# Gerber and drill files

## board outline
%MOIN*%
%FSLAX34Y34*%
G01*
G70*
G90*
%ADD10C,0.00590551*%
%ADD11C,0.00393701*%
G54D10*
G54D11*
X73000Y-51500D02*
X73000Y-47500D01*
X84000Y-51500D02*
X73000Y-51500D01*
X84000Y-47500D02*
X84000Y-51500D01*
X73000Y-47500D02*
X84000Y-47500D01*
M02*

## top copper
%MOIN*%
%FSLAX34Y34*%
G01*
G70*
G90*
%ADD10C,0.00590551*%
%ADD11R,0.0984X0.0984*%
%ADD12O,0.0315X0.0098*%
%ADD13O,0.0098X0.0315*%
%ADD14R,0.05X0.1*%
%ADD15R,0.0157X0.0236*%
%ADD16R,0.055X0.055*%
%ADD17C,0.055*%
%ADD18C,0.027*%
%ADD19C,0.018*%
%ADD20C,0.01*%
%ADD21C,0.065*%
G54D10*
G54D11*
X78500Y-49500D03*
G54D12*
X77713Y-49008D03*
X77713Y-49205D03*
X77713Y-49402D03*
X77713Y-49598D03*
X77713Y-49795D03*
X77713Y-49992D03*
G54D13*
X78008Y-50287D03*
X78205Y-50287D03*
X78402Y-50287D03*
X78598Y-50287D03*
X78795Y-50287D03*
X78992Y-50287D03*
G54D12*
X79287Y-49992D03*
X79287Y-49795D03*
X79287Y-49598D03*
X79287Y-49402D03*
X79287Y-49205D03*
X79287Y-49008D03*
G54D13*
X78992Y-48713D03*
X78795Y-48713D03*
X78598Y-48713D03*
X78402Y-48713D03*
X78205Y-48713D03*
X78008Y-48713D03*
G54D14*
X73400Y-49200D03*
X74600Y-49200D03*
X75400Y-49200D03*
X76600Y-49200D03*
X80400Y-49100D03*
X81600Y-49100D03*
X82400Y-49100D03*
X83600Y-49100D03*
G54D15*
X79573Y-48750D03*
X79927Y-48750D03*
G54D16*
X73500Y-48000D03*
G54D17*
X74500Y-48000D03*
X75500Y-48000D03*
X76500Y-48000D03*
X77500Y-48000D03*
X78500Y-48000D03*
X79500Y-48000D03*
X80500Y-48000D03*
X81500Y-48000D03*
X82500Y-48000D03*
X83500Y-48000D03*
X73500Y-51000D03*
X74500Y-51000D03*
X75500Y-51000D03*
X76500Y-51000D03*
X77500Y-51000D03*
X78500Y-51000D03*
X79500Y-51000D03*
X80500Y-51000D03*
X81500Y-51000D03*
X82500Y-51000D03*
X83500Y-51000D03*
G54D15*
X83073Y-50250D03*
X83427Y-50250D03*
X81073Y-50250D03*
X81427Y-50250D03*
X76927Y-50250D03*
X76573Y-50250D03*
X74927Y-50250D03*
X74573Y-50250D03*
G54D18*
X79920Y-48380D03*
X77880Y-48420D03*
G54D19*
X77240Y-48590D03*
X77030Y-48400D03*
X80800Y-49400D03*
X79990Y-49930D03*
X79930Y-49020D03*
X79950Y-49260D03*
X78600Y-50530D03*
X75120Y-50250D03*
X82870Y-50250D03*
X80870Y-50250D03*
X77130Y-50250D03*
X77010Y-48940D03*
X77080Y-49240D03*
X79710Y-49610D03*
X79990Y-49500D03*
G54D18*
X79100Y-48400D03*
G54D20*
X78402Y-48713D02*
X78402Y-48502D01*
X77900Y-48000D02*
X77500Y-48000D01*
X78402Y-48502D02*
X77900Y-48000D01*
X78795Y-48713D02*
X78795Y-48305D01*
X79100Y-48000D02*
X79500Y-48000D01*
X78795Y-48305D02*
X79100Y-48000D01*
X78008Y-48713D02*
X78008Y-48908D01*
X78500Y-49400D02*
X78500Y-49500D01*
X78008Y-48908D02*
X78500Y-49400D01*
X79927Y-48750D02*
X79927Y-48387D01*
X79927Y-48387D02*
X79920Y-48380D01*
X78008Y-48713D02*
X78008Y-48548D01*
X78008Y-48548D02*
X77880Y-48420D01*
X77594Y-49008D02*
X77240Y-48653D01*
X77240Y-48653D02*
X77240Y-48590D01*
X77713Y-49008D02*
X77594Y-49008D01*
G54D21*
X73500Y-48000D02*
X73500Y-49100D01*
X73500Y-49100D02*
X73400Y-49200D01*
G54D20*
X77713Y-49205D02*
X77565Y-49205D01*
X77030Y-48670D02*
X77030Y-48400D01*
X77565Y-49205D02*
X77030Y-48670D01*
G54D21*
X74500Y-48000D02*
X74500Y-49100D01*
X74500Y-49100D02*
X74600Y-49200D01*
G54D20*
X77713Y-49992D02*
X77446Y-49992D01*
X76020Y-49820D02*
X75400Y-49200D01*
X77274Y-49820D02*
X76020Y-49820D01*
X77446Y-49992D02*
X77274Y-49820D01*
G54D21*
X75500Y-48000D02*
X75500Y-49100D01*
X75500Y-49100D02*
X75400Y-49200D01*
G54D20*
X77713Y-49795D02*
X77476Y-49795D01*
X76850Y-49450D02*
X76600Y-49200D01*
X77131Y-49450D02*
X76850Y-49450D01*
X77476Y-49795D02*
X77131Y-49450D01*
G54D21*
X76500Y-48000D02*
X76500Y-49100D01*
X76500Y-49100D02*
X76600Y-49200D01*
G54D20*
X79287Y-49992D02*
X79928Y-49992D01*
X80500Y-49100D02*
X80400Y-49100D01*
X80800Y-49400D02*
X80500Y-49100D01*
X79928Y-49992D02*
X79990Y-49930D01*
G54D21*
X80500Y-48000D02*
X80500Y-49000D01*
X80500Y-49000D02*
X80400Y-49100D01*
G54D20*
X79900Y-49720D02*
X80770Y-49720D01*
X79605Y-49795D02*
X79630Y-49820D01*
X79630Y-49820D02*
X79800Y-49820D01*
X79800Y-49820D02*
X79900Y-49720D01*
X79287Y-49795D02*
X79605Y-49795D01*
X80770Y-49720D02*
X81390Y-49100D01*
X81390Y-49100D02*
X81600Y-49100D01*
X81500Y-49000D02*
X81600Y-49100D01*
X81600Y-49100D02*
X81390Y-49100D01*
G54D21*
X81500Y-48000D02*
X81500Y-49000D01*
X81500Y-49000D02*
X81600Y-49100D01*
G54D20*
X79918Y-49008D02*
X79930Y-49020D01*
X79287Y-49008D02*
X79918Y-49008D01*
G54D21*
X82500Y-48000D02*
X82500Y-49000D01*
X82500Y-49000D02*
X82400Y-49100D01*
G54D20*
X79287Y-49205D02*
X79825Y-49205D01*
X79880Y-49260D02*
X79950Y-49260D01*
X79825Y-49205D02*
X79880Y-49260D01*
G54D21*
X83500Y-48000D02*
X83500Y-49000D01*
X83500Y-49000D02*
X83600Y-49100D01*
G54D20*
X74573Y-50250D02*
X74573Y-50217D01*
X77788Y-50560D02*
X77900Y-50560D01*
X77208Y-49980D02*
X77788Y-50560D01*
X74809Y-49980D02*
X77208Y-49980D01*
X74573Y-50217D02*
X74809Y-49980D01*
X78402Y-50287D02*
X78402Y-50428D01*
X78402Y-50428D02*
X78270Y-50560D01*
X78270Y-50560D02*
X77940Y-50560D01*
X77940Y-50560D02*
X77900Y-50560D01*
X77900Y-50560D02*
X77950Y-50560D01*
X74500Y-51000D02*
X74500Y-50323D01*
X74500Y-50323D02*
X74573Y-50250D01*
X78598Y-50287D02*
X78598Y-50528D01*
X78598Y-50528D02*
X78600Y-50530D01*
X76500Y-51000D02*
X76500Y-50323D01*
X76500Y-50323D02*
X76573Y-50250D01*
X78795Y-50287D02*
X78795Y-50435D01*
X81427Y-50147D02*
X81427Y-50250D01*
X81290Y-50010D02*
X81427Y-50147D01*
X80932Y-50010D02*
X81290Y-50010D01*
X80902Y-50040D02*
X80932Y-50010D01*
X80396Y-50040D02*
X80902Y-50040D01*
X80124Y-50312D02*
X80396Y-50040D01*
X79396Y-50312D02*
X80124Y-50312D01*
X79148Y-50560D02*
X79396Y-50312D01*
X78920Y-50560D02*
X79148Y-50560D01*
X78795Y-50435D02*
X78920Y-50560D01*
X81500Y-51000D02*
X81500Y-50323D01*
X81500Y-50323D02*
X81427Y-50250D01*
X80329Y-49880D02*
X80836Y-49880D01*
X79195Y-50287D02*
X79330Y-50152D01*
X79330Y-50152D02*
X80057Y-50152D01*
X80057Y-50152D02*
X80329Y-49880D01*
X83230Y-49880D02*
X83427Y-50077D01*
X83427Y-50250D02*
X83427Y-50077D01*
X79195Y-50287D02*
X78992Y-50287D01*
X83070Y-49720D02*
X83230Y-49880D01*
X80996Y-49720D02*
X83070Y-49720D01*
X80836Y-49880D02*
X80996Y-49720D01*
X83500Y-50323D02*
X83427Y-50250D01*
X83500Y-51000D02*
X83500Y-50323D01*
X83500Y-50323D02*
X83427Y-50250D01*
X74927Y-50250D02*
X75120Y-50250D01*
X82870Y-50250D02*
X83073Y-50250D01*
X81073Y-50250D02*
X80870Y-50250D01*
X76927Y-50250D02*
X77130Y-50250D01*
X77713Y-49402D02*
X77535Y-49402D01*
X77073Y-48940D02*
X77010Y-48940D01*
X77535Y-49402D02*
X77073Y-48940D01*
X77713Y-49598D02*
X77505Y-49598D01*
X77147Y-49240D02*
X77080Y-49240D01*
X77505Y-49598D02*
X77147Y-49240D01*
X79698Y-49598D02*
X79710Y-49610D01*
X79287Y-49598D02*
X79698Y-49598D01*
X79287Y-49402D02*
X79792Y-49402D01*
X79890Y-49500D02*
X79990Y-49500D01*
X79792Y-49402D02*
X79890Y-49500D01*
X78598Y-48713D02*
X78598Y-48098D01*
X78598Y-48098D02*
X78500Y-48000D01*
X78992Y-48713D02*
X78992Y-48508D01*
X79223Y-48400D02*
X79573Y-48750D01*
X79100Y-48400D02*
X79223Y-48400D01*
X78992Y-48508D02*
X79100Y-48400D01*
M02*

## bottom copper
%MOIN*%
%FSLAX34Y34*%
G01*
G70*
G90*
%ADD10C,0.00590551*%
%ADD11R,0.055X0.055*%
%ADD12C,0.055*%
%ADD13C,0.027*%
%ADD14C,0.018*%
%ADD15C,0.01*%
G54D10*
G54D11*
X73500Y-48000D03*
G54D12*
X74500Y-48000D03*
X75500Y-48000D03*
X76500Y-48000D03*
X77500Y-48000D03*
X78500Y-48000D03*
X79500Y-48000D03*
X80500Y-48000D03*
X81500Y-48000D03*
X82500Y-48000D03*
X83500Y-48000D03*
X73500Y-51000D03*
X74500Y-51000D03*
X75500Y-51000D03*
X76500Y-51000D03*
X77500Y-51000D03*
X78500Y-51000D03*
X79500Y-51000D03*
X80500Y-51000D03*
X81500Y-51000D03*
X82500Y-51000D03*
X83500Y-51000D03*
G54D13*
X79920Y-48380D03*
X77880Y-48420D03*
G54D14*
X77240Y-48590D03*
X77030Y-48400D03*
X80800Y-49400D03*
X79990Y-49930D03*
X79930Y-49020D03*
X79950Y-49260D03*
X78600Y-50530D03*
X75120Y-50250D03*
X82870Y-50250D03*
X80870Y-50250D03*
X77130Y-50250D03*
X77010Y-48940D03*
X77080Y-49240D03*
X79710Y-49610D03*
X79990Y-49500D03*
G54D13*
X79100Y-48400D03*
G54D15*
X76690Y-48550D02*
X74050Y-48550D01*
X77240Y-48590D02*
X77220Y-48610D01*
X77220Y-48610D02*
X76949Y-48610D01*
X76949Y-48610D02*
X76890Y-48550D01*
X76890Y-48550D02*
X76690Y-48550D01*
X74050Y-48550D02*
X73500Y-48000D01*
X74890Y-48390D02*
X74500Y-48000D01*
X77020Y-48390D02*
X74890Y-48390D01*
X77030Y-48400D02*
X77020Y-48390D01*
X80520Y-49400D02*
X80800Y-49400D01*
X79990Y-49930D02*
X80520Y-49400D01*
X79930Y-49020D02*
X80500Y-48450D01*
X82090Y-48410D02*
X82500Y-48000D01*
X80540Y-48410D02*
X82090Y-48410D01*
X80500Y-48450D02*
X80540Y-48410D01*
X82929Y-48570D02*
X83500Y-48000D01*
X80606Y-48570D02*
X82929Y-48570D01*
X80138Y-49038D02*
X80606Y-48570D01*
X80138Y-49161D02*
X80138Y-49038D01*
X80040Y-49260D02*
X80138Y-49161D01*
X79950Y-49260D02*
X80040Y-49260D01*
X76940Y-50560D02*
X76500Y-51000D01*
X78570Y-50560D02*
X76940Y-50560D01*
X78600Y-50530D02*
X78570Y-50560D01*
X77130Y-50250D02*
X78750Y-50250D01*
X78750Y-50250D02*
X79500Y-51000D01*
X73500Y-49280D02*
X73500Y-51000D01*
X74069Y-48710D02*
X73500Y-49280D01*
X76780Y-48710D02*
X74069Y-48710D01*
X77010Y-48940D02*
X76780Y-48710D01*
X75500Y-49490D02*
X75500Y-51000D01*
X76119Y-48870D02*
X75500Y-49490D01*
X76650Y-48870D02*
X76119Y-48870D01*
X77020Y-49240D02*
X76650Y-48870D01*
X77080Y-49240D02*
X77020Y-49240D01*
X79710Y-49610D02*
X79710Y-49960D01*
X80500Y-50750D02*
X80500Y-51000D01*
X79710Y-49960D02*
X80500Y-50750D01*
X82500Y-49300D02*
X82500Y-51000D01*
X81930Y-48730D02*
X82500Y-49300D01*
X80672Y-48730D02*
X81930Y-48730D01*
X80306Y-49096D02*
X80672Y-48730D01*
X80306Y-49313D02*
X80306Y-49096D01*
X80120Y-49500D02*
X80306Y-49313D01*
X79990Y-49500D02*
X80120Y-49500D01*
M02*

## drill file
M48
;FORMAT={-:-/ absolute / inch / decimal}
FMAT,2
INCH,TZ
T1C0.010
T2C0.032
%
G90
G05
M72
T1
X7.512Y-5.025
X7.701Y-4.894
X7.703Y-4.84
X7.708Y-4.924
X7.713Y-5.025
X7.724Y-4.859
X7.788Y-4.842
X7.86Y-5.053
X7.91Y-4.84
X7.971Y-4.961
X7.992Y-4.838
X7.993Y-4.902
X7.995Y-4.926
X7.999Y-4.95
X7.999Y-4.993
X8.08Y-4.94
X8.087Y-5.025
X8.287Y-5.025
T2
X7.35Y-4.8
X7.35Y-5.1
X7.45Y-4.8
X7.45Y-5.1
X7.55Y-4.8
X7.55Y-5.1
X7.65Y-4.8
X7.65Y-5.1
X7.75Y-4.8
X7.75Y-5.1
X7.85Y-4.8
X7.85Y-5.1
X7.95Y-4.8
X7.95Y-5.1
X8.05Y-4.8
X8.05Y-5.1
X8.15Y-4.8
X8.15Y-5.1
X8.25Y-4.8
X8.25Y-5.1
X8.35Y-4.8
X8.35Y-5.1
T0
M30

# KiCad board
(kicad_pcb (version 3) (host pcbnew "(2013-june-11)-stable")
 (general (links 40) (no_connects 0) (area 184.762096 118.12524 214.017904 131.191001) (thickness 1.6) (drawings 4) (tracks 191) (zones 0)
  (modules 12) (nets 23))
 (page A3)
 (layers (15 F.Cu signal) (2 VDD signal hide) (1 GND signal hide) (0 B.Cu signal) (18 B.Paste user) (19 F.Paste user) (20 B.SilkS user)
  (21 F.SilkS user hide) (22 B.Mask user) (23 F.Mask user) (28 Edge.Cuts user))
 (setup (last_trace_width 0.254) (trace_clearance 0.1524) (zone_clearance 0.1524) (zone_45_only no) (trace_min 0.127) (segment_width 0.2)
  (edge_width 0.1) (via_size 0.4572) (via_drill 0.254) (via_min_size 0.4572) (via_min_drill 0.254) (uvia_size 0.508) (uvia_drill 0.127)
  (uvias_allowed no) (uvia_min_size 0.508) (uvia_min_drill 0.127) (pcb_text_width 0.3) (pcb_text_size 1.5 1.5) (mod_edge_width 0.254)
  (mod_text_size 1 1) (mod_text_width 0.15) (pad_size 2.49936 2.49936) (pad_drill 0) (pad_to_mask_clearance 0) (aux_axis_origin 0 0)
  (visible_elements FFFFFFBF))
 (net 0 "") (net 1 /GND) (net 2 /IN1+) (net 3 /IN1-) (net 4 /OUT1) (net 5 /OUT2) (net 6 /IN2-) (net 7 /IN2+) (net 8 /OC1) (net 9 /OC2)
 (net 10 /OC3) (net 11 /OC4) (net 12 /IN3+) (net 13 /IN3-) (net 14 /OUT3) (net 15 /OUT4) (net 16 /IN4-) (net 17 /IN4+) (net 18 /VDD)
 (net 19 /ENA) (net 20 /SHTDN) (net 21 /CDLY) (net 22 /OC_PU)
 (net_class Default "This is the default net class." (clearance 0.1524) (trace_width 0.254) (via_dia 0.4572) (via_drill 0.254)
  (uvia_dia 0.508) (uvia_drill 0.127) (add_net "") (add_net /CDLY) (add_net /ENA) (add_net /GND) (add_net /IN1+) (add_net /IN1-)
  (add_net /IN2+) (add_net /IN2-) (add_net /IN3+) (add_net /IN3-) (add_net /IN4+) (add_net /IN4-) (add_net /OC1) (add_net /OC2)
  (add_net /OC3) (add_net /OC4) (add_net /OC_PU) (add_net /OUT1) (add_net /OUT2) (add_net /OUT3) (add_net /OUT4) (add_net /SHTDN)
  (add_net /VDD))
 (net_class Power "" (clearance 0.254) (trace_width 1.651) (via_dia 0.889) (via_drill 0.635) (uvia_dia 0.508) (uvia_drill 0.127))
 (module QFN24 (layer F.Cu) (at 199.39 125.73) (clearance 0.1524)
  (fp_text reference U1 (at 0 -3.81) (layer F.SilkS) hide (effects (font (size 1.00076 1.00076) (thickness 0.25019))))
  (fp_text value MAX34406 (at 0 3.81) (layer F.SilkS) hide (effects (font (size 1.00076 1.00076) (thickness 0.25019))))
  (pad 25 smd rect (at 0 0 270) (size 2.49936 2.49936) (layers F.Cu F.Paste F.Mask) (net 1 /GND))
  (pad 1 smd oval (at -1.99898 -1.24968) (size 0.8001 0.24892) (layers F.Cu F.Paste F.Mask) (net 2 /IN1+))
  (pad 2 smd oval (at -1.99898 -0.7493) (size 0.8001 0.24892) (layers F.Cu F.Paste F.Mask) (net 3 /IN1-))
  (pad 3 smd oval (at -1.99898 -0.24892) (size 0.8001 0.24892) (layers F.Cu F.Paste F.Mask) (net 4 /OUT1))
  (pad 4 smd oval (at -1.99898 0.24892) (size 0.8001 0.24892) (layers F.Cu F.Paste F.Mask) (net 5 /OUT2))
  (pad 5 smd oval (at -1.99898 0.7493) (size 0.8001 0.24892) (layers F.Cu F.Paste F.Mask) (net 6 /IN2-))
  (pad 6 smd oval (at -1.99898 1.24968) (size 0.8001 0.24892) (layers F.Cu F.Paste F.Mask) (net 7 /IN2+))
  (pad 7 smd oval (at -1.24968 1.99898 90) (size 0.8001 0.24892) (layers F.Cu F.Paste F.Mask))
  (pad 8 smd oval (at -0.7493 1.99898 90) (size 0.8001 0.24892) (layers F.Cu F.Paste F.Mask))
  (pad 9 smd oval (at -0.24892 1.99898 90) (size 0.8001 0.24892) (layers F.Cu F.Paste F.Mask) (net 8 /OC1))
  (pad 10 smd oval (at 0.24892 1.99898 90) (size 0.8001 0.24892) (layers F.Cu F.Paste F.Mask) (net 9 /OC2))
  (pad 11 smd oval (at 0.7493 1.99898 90) (size 0.8001 0.24892) (layers F.Cu F.Paste F.Mask) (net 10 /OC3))
  (pad 12 smd oval (at 1.24968 1.99898 90) (size 0.8001 0.24892) (layers F.Cu F.Paste F.Mask) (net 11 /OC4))
  (pad 13 smd oval (at 1.99898 1.24968 180) (size 0.8001 0.24892) (layers F.Cu F.Paste F.Mask) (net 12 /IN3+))
  (pad 14 smd oval (at 1.99898 0.7493 180) (size 0.8001 0.24892) (layers F.Cu F.Paste F.Mask) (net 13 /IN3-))
  (pad 15 smd oval (at 1.99898 0.24892 180) (size 0.8001 0.24892) (layers F.Cu F.Paste F.Mask) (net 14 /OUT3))
  (pad 16 smd oval (at 1.99898 -0.24892 180) (size 0.8001 0.24892) (layers F.Cu F.Paste F.Mask) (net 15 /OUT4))
  (pad 17 smd oval (at 1.99898 -0.7493 180) (size 0.8001 0.24892) (layers F.Cu F.Paste F.Mask) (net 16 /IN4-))
  (pad 18 smd oval (at 1.99898 -1.24968 180) (size 0.8001 0.24892) (layers F.Cu F.Paste F.Mask) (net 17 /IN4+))
  (pad 19 smd oval (at 1.24968 -1.99898 270) (size 0.8001 0.24892) (layers F.Cu F.Paste F.Mask) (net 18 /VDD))
  (pad 20 smd oval (at 0.7493 -1.99898 270) (size 0.8001 0.24892) (layers F.Cu F.Paste F.Mask) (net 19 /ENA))
  (pad 21 smd oval (at 0.24892 -1.99898 270) (size 0.8001 0.24892) (layers F.Cu F.Paste F.Mask) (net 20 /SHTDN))
  (pad 22 smd oval (at -0.24892 -1.99898 270) (size 0.8001 0.24892) (layers F.Cu F.Paste F.Mask) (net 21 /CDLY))
  (pad 23 smd oval (at -0.7493 -1.99898 270) (size 0.8001 0.24892) (layers F.Cu F.Paste F.Mask))
  (pad 24 smd oval (at -1.24968 -1.99898 270) (size 0.8001 0.24892) (layers F.Cu F.Paste F.Mask) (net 1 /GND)))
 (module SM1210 (layer F.Cu) (at 187.96 124.968)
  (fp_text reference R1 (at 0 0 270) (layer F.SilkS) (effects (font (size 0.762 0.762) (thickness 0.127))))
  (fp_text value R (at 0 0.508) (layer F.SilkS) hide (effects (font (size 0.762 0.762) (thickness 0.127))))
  (pad 1 smd rect (at -1.524 0) (size 1.27 2.54) (layers F.Cu F.Paste F.Mask) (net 2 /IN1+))
  (pad 2 smd rect (at 1.524 0) (size 1.27 2.54) (layers F.Cu F.Paste F.Mask) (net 3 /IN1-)))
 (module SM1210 (layer F.Cu) (at 193.04 124.968)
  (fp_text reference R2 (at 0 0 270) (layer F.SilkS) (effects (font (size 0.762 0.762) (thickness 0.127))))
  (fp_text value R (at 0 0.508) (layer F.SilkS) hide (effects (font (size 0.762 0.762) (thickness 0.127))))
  (pad 1 smd rect (at -1.524 0) (size 1.27 2.54) (layers F.Cu F.Paste F.Mask) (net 7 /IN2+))
  (pad 2 smd rect (at 1.524 0) (size 1.27 2.54) (layers F.Cu F.Paste F.Mask) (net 6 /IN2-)))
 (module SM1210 (layer F.Cu) (at 205.74 124.714)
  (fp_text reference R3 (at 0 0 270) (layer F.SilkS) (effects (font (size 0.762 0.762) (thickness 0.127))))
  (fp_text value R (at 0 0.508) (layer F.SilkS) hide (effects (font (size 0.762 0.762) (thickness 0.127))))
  (pad 1 smd rect (at -1.524 0) (size 1.27 2.54) (layers F.Cu F.Paste F.Mask) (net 12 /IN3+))
  (pad 2 smd rect (at 1.524 0) (size 1.27 2.54) (layers F.Cu F.Paste F.Mask) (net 13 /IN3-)))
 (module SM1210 (layer F.Cu) (at 210.82 124.714)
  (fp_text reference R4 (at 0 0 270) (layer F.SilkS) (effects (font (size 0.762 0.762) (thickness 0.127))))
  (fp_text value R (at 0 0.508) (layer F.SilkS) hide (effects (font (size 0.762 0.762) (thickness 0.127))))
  (pad 1 smd rect (at -1.524 0) (size 1.27 2.54) (layers F.Cu F.Paste F.Mask) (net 17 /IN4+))
  (pad 2 smd rect (at 1.524 0) (size 1.27 2.54) (layers F.Cu F.Paste F.Mask) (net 16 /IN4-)))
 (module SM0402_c (layer F.Cu) (at 202.565 123.825)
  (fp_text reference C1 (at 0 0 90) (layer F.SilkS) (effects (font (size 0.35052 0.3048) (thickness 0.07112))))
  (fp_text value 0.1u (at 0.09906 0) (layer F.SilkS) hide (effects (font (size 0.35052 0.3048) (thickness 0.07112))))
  (pad 1 smd rect (at -0.44958 0) (size 0.39878 0.59944) (layers F.Cu F.Paste F.Mask) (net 18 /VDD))
  (pad 2 smd rect (at 0.44958 0) (size 0.39878 0.59944) (layers F.Cu F.Paste F.Mask) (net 1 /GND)))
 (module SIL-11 (layer F.Cu) (at 200.66 121.92)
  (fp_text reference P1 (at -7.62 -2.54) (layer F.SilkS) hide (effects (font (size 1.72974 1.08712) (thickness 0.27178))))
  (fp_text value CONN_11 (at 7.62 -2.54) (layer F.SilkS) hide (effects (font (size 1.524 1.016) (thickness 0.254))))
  (pad 1 thru_hole rect (at -13.97 0) (size 1.397 1.397) (drill 0.8128) (layers *.Cu *.Mask F.SilkS) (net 2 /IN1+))
  (pad 2 thru_hole circle (at -11.43 0) (size 1.397 1.397) (drill 0.8128) (layers *.Cu *.Mask F.SilkS) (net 3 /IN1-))
  (pad 3 thru_hole circle (at -8.89 0) (size 1.397 1.397) (drill 0.8128) (layers *.Cu *.Mask F.SilkS) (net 7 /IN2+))
  (pad 4 thru_hole circle (at -6.35 0) (size 1.397 1.397) (drill 0.8128) (layers *.Cu *.Mask F.SilkS) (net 6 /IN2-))
  (pad 5 thru_hole circle (at -3.81 0) (size 1.397 1.397) (drill 0.8128) (layers *.Cu *.Mask F.SilkS) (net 21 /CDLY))
  (pad 6 thru_hole circle (at -1.27 0) (size 1.397 1.397) (drill 0.8128) (layers *.Cu *.Mask F.SilkS) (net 20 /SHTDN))
  (pad 7 thru_hole circle (at 1.27 0) (size 1.397 1.397) (drill 0.8128) (layers *.Cu *.Mask F.SilkS) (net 19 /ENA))
  (pad 8 thru_hole circle (at 3.81 0) (size 1.397 1.397) (drill 0.8128) (layers *.Cu *.Mask F.SilkS) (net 12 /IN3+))
  (pad 9 thru_hole circle (at 6.35 0) (size 1.397 1.397) (drill 0.8128) (layers *.Cu *.Mask F.SilkS) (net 13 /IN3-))
  (pad 10 thru_hole circle (at 8.89 0) (size 1.397 1.397) (drill 0.8128) (layers *.Cu *.Mask F.SilkS) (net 17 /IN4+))
  (pad 11 thru_hole circle (at 11.43 0) (size 1.397 1.397) (drill 0.8128) (layers *.Cu *.Mask F.SilkS) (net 16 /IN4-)))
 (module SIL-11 (layer F.Cu) (at 200.66 129.54)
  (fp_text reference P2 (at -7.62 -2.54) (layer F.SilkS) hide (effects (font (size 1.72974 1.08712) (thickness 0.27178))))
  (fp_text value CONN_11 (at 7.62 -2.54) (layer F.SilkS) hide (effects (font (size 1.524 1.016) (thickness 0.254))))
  (pad 1 thru_hole circle (at -13.97 0) (size 1.397 1.397) (drill 0.8128) (layers *.Cu *.Mask F.SilkS) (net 4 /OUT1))
  (pad 2 thru_hole circle (at -11.43 0) (size 1.397 1.397) (drill 0.8128) (layers *.Cu *.Mask F.SilkS) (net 8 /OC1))
  (pad 3 thru_hole circle (at -8.89 0) (size 1.397 1.397) (drill 0.8128) (layers *.Cu *.Mask F.SilkS) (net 5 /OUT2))
  (pad 4 thru_hole circle (at -6.35 0) (size 1.397 1.397) (drill 0.8128) (layers *.Cu *.Mask F.SilkS) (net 9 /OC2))
  (pad 5 thru_hole circle (at -3.81 0) (size 1.397 1.397) (drill 0.8128) (layers *.Cu *.Mask F.SilkS) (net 1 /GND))
  (pad 6 thru_hole circle (at -1.27 0) (size 1.397 1.397) (drill 0.8128) (layers *.Cu *.Mask F.SilkS) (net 18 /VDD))
  (pad 7 thru_hole circle (at 1.27 0) (size 1.397 1.397) (drill 0.8128) (layers *.Cu *.Mask F.SilkS) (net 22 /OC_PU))
  (pad 8 thru_hole circle (at 3.81 0) (size 1.397 1.397) (drill 0.8128) (layers *.Cu *.Mask F.SilkS) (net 14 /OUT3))
  (pad 9 thru_hole circle (at 6.35 0) (size 1.397 1.397) (drill 0.8128) (layers *.Cu *.Mask F.SilkS) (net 10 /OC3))
  (pad 10 thru_hole circle (at 8.89 0) (size 1.397 1.397) (drill 0.8128) (layers *.Cu *.Mask F.SilkS) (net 15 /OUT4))
  (pad 11 thru_hole circle (at 11.43 0) (size 1.397 1.397) (drill 0.8128) (layers *.Cu *.Mask F.SilkS) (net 11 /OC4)))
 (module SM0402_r (layer F.Cu) (at 211.455 127.635)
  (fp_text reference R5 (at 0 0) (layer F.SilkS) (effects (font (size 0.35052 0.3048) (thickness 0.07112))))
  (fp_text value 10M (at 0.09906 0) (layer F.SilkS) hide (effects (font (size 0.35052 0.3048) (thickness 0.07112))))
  (pad 1 smd rect (at -0.44958 0) (size 0.39878 0.59944) (layers F.Cu F.Paste F.Mask) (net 22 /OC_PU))
  (pad 2 smd rect (at 0.44958 0) (size 0.39878 0.59944) (layers F.Cu F.Paste F.Mask) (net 11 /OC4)))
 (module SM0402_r (layer F.Cu) (at 206.375 127.635)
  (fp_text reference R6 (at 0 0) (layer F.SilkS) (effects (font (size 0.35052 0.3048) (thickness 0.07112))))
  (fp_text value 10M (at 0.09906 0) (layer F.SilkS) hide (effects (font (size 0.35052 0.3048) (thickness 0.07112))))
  (pad 1 smd rect (at -0.44958 0) (size 0.39878 0.59944) (layers F.Cu F.Paste F.Mask) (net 22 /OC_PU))
  (pad 2 smd rect (at 0.44958 0) (size 0.39878 0.59944) (layers F.Cu F.Paste F.Mask) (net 10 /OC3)))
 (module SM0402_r (layer F.Cu) (at 194.945 127.635 180)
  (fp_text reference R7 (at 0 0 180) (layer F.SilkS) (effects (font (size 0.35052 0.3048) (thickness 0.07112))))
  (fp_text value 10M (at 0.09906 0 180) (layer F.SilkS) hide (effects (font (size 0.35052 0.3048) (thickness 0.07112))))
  (pad 1 smd rect (at -0.44958 0 180) (size 0.39878 0.59944) (layers F.Cu F.Paste F.Mask) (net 22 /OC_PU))
  (pad 2 smd rect (at 0.44958 0 180) (size 0.39878 0.59944) (layers F.Cu F.Paste F.Mask) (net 9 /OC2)))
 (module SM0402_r (layer F.Cu) (at 189.865 127.635 180)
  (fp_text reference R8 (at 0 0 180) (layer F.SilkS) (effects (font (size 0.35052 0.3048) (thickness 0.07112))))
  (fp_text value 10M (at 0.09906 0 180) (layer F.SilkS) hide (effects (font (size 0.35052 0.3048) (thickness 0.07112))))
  (pad 1 smd rect (at -0.44958 0 180) (size 0.39878 0.59944) (layers F.Cu F.Paste F.Mask) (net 22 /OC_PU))
  (pad 2 smd rect (at 0.44958 0 180) (size 0.39878 0.59944) (layers F.Cu F.Paste F.Mask) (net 8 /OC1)))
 (gr_line (start 185.42 130.81) (end 185.42 120.65) (angle 90) (layer Edge.Cuts) (width 0.1))
 (gr_line (start 213.36 130.81) (end 185.42 130.81) (angle 90) (layer Edge.Cuts) (width 0.1))
 (gr_line (start 213.36 120.65) (end 213.36 130.81) (angle 90) (layer Edge.Cuts) (width 0.1))
 (gr_line (start 185.42 120.65) (end 213.36 120.65) (angle 90) (layer Edge.Cuts) (width 0.1))
 (segment (start 199.14108 123.73102) (end 199.14108 123.19508) (width 0.254) (layer F.Cu) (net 21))
 (segment (start 197.866 121.92) (end 196.85 121.92) (width 0.254) (layer F.Cu) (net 21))
 (segment (start 199.14108 123.19508) (end 197.866 121.92) (width 0.254) (layer F.Cu) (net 21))
 (segment (start 200.1393 123.73102) (end 200.1393 122.6947) (width 0.254) (layer F.Cu) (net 19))
 (segment (start 200.914 121.92) (end 201.93 121.92) (width 0.254) (layer F.Cu) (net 19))
 (segment (start 200.1393 122.6947) (end 200.914 121.92) (width 0.254) (layer F.Cu) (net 19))
 (segment (start 198.14032 123.73102) (end 198.14032 124.22632) (width 0.254) (layer F.Cu) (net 1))
 (segment (start 199.39 125.476) (end 199.39 125.73) (width 0.254) (layer F.Cu) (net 1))
 (segment (start 198.14032 124.22632) (end 199.39 125.476) (width 0.254) (layer F.Cu) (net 1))
 (segment (start 203.01458 123.825) (end 203.01458 122.90298) (width 0.254) (layer F.Cu) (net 1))
 (via (at 202.9968 122.8852) (size 0.6858) (layers F.Cu B.Cu) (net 1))
 (segment (start 203.01458 122.90298) (end 202.9968 122.8852) (width 0.254) (layer F.Cu) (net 1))
 (segment (start 198.14032 123.73102) (end 198.14032 123.31192) (width 0.254) (layer F.Cu) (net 1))
 (via (at 197.8152 122.9868) (size 0.6858) (layers F.Cu B.Cu) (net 1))
 (segment (start 198.14032 123.31192) (end 197.8152 122.9868) (width 0.254) (layer F.Cu) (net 1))
 (segment (start 194.7926 123.317002) (end 188.087002 123.317002) (width 0.254) (layer B.Cu) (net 2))
 (segment (start 197.08946 124.48032) (end 196.1896 123.58046) (width 0.254) (layer F.Cu) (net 2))
 (segment (start 196.1896 123.58046) (end 196.1896 123.4186) (width 0.254) (layer F.Cu) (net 2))
 (via (at 196.1896 123.4186) (size 0.4572) (layers F.Cu B.Cu) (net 2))
 (segment (start 196.1896 123.4186) (end 196.1388 123.4694) (width 0.254) (layer B.Cu) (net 2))
 (segment (start 196.1388 123.4694) (end 195.452998 123.4694) (width 0.254) (layer B.Cu) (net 2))
 (segment (start 195.452998 123.4694) (end 195.3006 123.317002) (width 0.254) (layer B.Cu) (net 2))
 (segment (start 195.3006 123.317002) (end 194.7926 123.317002) (width 0.254) (layer B.Cu) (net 2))
 (segment (start 197.39102 124.48032) (end 197.08946 124.48032) (width 0.254) (layer F.Cu) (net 2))
 (segment (start 188.087002 123.317002) (end 186.69 121.92) (width 0.254) (layer B.Cu) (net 2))
 (segment (start 186.69 121.92) (end 186.69 124.714) (width 1.651) (layer F.Cu) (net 2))
 (segment (start 186.69 124.714) (end 186.436 124.968) (width 1.651) (layer F.Cu) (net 2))
 (segment (start 197.39102 124.9807) (end 197.0151 124.9807) (width 0.254) (layer F.Cu) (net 3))
 (segment (start 190.2206 122.9106) (end 189.23 121.92) (width 0.254) (layer B.Cu) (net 3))
 (segment (start 195.6308 122.9106) (end 190.2206 122.9106) (width 0.254) (layer B.Cu) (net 3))
 (segment (start 195.6562 122.936) (end 195.6308 122.9106) (width 0.254) (layer B.Cu) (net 3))
 (via (at 195.6562 122.936) (size 0.4572) (layers F.Cu B.Cu) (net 3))
 (segment (start 195.6562 123.6218) (end 195.6562 122.936) (width 0.254) (layer F.Cu) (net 3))
 (segment (start 197.0151 124.9807) (end 195.6562 123.6218) (width 0.254) (layer F.Cu) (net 3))
 (segment (start 189.23 121.92) (end 189.23 124.714) (width 1.651) (layer F.Cu) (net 3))
 (segment (start 189.23 124.714) (end 189.484 124.968) (width 1.651) (layer F.Cu) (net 3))
 (segment (start 197.39102 126.97968) (end 196.71512 126.97968) (width 0.254) (layer F.Cu) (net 7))
 (segment (start 193.0908 126.5428) (end 191.516 124.968) (width 0.254) (layer F.Cu) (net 7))
 (segment (start 196.27824 126.5428) (end 193.0908 126.5428) (width 0.254) (layer F.Cu) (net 7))
 (segment (start 196.71512 126.97968) (end 196.27824 126.5428) (width 0.254) (layer F.Cu) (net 7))
 (segment (start 191.77 121.92) (end 191.77 124.714) (width 1.651) (layer F.Cu) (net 7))
 (segment (start 191.77 124.714) (end 191.516 124.968) (width 1.651) (layer F.Cu) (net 7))
 (segment (start 197.39102 126.4793) (end 196.78948 126.4793) (width 0.254) (layer F.Cu) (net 6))
 (segment (start 195.199 125.603) (end 194.564 124.968) (width 0.254) (layer F.Cu) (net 6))
 (segment (start 195.91318 125.603) (end 195.199 125.603) (width 0.254) (layer F.Cu) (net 6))
 (segment (start 196.78948 126.4793) (end 195.91318 125.603) (width 0.254) (layer F.Cu) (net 6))
 (segment (start 194.31 121.92) (end 194.31 124.714) (width 1.651) (layer F.Cu) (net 6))
 (segment (start 194.31 124.714) (end 194.564 124.968) (width 1.651) (layer F.Cu) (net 6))
 (segment (start 201.38898 126.97968) (end 203.01712 126.97968) (width 0.254) (layer F.Cu) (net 12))
 (segment (start 204.47 124.714) (end 204.216 124.714) (width 0.254) (layer F.Cu) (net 12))
 (segment (start 205.232 125.476) (end 204.47 124.714) (width 0.254) (layer F.Cu) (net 12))
 (via (at 205.232 125.476) (size 0.4572) (layers F.Cu B.Cu) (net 12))
 (segment (start 204.5208 125.476) (end 205.232 125.476) (width 0.254) (layer B.Cu) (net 12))
 (segment (start 203.1746 126.8222) (end 204.5208 125.476) (width 0.254) (layer B.Cu) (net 12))
 (via (at 203.1746 126.8222) (size 0.4572) (layers F.Cu B.Cu) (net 12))
 (segment (start 203.01712 126.97968) (end 203.1746 126.8222) (width 0.254) (layer F.Cu) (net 12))
 (segment (start 204.47 121.92) (end 204.47 124.46) (width 1.651) (layer F.Cu) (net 12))
 (segment (start 204.47 124.46) (end 204.216 124.714) (width 1.651) (layer F.Cu) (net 12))
 (segment (start 202.946 126.2888) (end 205.1558 126.2888) (width 0.254) (layer F.Cu) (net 13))
 (segment (start 202.1967 126.4793) (end 202.2602 126.5428) (width 0.254) (layer F.Cu) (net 13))
 (segment (start 202.2602 126.5428) (end 202.692 126.5428) (width 0.254) (layer F.Cu) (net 13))
 (segment (start 202.692 126.5428) (end 202.946 126.2888) (width 0.254) (layer F.Cu) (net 13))
 (segment (start 201.38898 126.4793) (end 202.1967 126.4793) (width 0.254) (layer F.Cu) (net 13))
 (segment (start 205.1558 126.2888) (end 206.7306 124.714) (width 0.254) (layer F.Cu) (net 13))
 (segment (start 206.7306 124.714) (end 207.264 124.714) (width 0.254) (layer F.Cu) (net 13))
 (segment (start 207.01 124.46) (end 207.264 124.714) (width 0.254) (layer F.Cu) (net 13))
 (segment (start 207.264 124.714) (end 206.7306 124.714) (width 0.254) (layer F.Cu) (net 13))
 (segment (start 207.01 121.92) (end 207.01 124.46) (width 1.651) (layer F.Cu) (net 13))
 (segment (start 207.01 124.46) (end 207.264 124.714) (width 1.651) (layer F.Cu) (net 13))
 (segment (start 203.0222 124.5108) (end 204.47 123.063) (width 0.254) (layer B.Cu) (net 17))
 (segment (start 202.99172 124.48032) (end 203.0222 124.5108) (width 0.254) (layer F.Cu) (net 17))
 (via (at 203.0222 124.5108) (size 0.4572) (layers F.Cu B.Cu) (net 17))
 (segment (start 201.38898 124.48032) (end 202.99172 124.48032) (width 0.254) (layer F.Cu) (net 17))
 (segment (start 208.5086 122.9614) (end 209.55 121.92) (width 0.254) (layer B.Cu) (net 17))
 (segment (start 204.5716 122.9614) (end 208.5086 122.9614) (width 0.254) (layer B.Cu) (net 17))
 (segment (start 204.47 123.063) (end 204.5716 122.9614) (width 0.254) (layer B.Cu) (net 17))
 (segment (start 209.55 121.92) (end 209.55 124.46) (width 1.651) (layer F.Cu) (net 17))
 (segment (start 209.55 124.46) (end 209.296 124.714) (width 1.651) (layer F.Cu) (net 17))
 (segment (start 201.38898 124.9807) (end 202.7555 124.9807) (width 0.254) (layer F.Cu) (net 16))
 (segment (start 210.642198 123.367802) (end 212.09 121.92) (width 0.254) (layer B.Cu) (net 16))
 (segment (start 204.739938 123.367802) (end 210.642198 123.367802) (width 0.254) (layer B.Cu) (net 16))
 (segment (start 203.55087 124.55687) (end 204.739938 123.367802) (width 0.254) (layer B.Cu) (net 16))
 (segment (start 203.55087 124.87113) (end 203.55087 124.55687) (width 0.254) (layer B.Cu) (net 16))
 (segment (start 203.3016 125.1204) (end 203.55087 124.87113) (width 0.254) (layer B.Cu) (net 16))
 (segment (start 203.073 125.1204) (end 203.3016 125.1204) (width 0.254) (layer B.Cu) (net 16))
 (via (at 203.073 125.1204) (size 0.4572) (layers F.Cu B.Cu) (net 16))
 (segment (start 202.8952 125.1204) (end 203.073 125.1204) (width 0.254) (layer F.Cu) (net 16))
 (segment (start 202.7555 124.9807) (end 202.8952 125.1204) (width 0.254) (layer F.Cu) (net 16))
 (segment (start 212.09 121.92) (end 212.09 124.46) (width 1.651) (layer F.Cu) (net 16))
 (segment (start 212.09 124.46) (end 212.344 124.714) (width 1.651) (layer F.Cu) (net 16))
 (segment (start 189.41542 127.635) (end 189.41542 127.55118) (width 0.254) (layer F.Cu) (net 8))
 (segment (start 197.5831 128.4224) (end 197.866 128.4224) (width 0.254) (layer F.Cu) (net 8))
 (segment (start 196.109902 126.949202) (end 197.5831 128.4224) (width 0.254) (layer F.Cu) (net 8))
 (segment (start 190.017398 126.949202) (end 196.109902 126.949202) (width 0.254) (layer F.Cu) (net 8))
 (segment (start 189.41542 127.55118) (end 190.017398 126.949202) (width 0.254) (layer F.Cu) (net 8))
 (segment (start 199.14108 127.72898) (end 199.14108 128.08712) (width 0.254) (layer F.Cu) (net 8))
 (segment (start 199.14108 128.08712) (end 198.8058 128.4224) (width 0.254) (layer F.Cu) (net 8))
 (segment (start 198.8058 128.4224) (end 197.9676 128.4224) (width 0.254) (layer F.Cu) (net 8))
 (segment (start 197.9676 128.4224) (end 197.866 128.4224) (width 0.254) (layer F.Cu) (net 8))
 (segment (start 197.866 128.4224) (end 197.993 128.4224) (width 0.254) (layer F.Cu) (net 8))
 (segment (start 189.23 129.54) (end 189.23 127.82042) (width 0.254) (layer F.Cu) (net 8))
 (segment (start 189.23 127.82042) (end 189.41542 127.635) (width 0.254) (layer F.Cu) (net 8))
 (segment (start 199.63892 127.72898) (end 199.63892 128.34112) (width 0.254) (layer F.Cu) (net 9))
 (segment (start 195.4276 128.4224) (end 194.31 129.54) (width 0.254) (layer B.Cu) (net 9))
 (segment (start 199.5678 128.4224) (end 195.4276 128.4224) (width 0.254) (layer B.Cu) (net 9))
 (segment (start 199.644 128.3462) (end 199.5678 128.4224) (width 0.254) (layer B.Cu) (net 9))
 (via (at 199.644 128.3462) (size 0.4572) (layers F.Cu B.Cu) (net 9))
 (segment (start 199.63892 128.34112) (end 199.644 128.3462) (width 0.254) (layer F.Cu) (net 9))
 (segment (start 194.31 129.54) (end 194.31 127.82042) (width 0.254) (layer F.Cu) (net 9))
 (segment (start 194.31 127.82042) (end 194.49542 127.635) (width 0.254) (layer F.Cu) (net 9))
 (segment (start 200.1393 127.72898) (end 200.1393 128.1049) (width 0.254) (layer F.Cu) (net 10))
 (segment (start 206.82458 127.37338) (end 206.82458 127.635) (width 0.254) (layer F.Cu) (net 10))
 (segment (start 206.4766 127.0254) (end 206.82458 127.37338) (width 0.254) (layer F.Cu) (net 10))
 (segment (start 205.56868 127.0254) (end 206.4766 127.0254) (width 0.254) (layer F.Cu) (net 10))
 (segment (start 205.492476 127.101604) (end 205.56868 127.0254) (width 0.254) (layer F.Cu) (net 10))
 (segment (start 204.206536 127.101604) (end 205.492476 127.101604) (width 0.254) (layer F.Cu) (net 10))
 (segment (start 203.515656 127.792484) (end 204.206536 127.101604) (width 0.254) (layer F.Cu) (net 10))
 (segment (start 201.666538 127.792484) (end 203.515656 127.792484) (width 0.254) (layer F.Cu) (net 10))
 (segment (start 201.036622 128.4224) (end 201.666538 127.792484) (width 0.254) (layer F.Cu) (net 10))
 (segment (start 200.4568 128.4224) (end 201.036622 128.4224) (width 0.254) (layer F.Cu) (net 10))
 (segment (start 200.1393 128.1049) (end 200.4568 128.4224) (width 0.254) (layer F.Cu) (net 10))
 (segment (start 207.01 129.54) (end 207.01 127.82042) (width 0.254) (layer F.Cu) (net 10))
 (segment (start 207.01 127.82042) (end 206.82458 127.635) (width 0.254) (layer F.Cu) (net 10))
 (segment (start 204.038198 126.695202) (end 205.324138 126.695202) (width 0.254) (layer F.Cu) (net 11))
 (segment (start 201.155302 127.72898) (end 201.4982 127.386082) (width 0.254) (layer F.Cu) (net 11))
 (segment (start 201.4982 127.386082) (end 203.347318 127.386082) (width 0.254) (layer F.Cu) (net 11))
 (segment (start 203.347318 127.386082) (end 204.038198 126.695202) (width 0.254) (layer F.Cu) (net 11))
 (segment (start 211.404202 126.695202) (end 211.90458 127.19558) (width 0.254) (layer F.Cu) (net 11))
 (segment (start 211.90458 127.635) (end 211.90458 127.19558) (width 0.254) (layer F.Cu) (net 11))
 (segment (start 201.155302 127.72898) (end 200.63968 127.72898) (width 0.254) (layer F.Cu) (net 11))
 (segment (start 210.9978 126.2888) (end 211.404202 126.695202) (width 0.254) (layer F.Cu) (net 11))
 (segment (start 205.73054 126.2888) (end 210.9978 126.2888) (width 0.254) (layer F.Cu) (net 11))
 (segment (start 205.324138 126.695202) (end 205.73054 126.2888) (width 0.254) (layer F.Cu) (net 11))
 (segment (start 212.09 127.82042) (end 211.90458 127.635) (width 0.254) (layer F.Cu) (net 11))
 (segment (start 212.09 129.54) (end 212.09 127.82042) (width 0.254) (layer F.Cu) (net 11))
 (segment (start 212.09 127.82042) (end 211.90458 127.635) (width 0.254) (layer F.Cu) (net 11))
 (segment (start 190.31458 127.635) (end 190.8048 127.635) (width 0.254) (layer F.Cu) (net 22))
 (via (at 190.8048 127.635) (size 0.4572) (layers F.Cu B.Cu) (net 22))
 (segment (start 190.8048 127.635) (end 195.9102 127.635) (width 0.254) (layer VDD) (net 22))
 (segment (start 205.4098 127.635) (end 210.4898 127.635) (width 0.254) (layer VDD) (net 22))
 (segment (start 210.4898 127.635) (end 211.00542 127.635) (width 0.254) (layer F.Cu) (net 22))
 (via (at 210.4898 127.635) (size 0.4572) (layers F.Cu B.Cu) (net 22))
 (segment (start 205.4098 127.635) (end 203.835 127.635) (width 0.254) (layer VDD) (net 22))
 (segment (start 203.835 127.635) (end 201.93 129.54) (width 0.254) (layer VDD) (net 22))
 (via (at 205.4098 127.635) (size 0.4572) (layers F.Cu B.Cu) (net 22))
 (segment (start 205.92542 127.635) (end 205.4098 127.635) (width 0.254) (layer F.Cu) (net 22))
 (segment (start 195.9102 127.635) (end 200.025 127.635) (width 0.254) (layer B.Cu) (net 22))
 (segment (start 200.025 127.635) (end 201.93 129.54) (width 0.254) (layer B.Cu) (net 22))
 (via (at 195.9102 127.635) (size 0.4572) (layers F.Cu B.Cu) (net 22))
 (segment (start 195.39458 127.635) (end 195.9102 127.635) (width 0.254) (layer F.Cu) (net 22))
 (segment (start 197.39102 125.48108) (end 196.94074 125.48108) (width 0.254) (layer F.Cu) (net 4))
 (segment (start 186.69 125.1712) (end 186.69 129.54) (width 0.254) (layer B.Cu) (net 4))
 (segment (start 188.137796 123.723404) (end 186.69 125.1712) (width 0.254) (layer B.Cu) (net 4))
 (segment (start 195.021204 123.723404) (end 188.137796 123.723404) (width 0.254) (layer B.Cu) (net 4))
 (segment (start 195.6054 124.3076) (end 195.021204 123.723404) (width 0.254) (layer B.Cu) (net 4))
 (via (at 195.6054 124.3076) (size 0.4572) (layers F.Cu B.Cu) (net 4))
 (segment (start 195.76726 124.3076) (end 195.6054 124.3076) (width 0.254) (layer F.Cu) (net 4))
 (segment (start 196.94074 125.48108) (end 195.76726 124.3076) (width 0.254) (layer F.Cu) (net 4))
 (segment (start 197.39102 125.97892) (end 196.86384 125.97892) (width 0.254) (layer F.Cu) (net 5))
 (segment (start 191.77 125.7046) (end 191.77 129.54) (width 0.254) (layer B.Cu) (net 5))
 (segment (start 193.344794 124.129806) (end 191.77 125.7046) (width 0.254) (layer B.Cu) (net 5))
 (segment (start 194.691006 124.129806) (end 193.344794 124.129806) (width 0.254) (layer B.Cu) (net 5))
 (segment (start 195.6308 125.0696) (end 194.691006 124.129806) (width 0.254) (layer B.Cu) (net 5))
 (segment (start 195.7832 125.0696) (end 195.6308 125.0696) (width 0.254) (layer B.Cu) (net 5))
 (via (at 195.7832 125.0696) (size 0.4572) (layers F.Cu B.Cu) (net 5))
 (segment (start 195.95452 125.0696) (end 195.7832 125.0696) (width 0.254) (layer F.Cu) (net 5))
 (segment (start 196.86384 125.97892) (end 195.95452 125.0696) (width 0.254) (layer F.Cu) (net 5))
 (segment (start 202.4634 126.0094) (end 202.4634 126.8984) (width 0.254) (layer B.Cu) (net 14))
 (segment (start 202.43292 125.97892) (end 202.4634 126.0094) (width 0.254) (layer F.Cu) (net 14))
 (via (at 202.4634 126.0094) (size 0.4572) (layers F.Cu B.Cu) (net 14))
 (segment (start 201.38898 125.97892) (end 202.43292 125.97892) (width 0.254) (layer F.Cu) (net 14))
 (segment (start 204.47 128.905) (end 204.47 129.54) (width 0.254) (layer B.Cu) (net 14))
 (segment (start 202.4634 126.8984) (end 204.47 128.905) (width 0.254) (layer B.Cu) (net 14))
 (segment (start 201.38898 125.48108) (end 202.67168 125.48108) (width 0.254) (layer F.Cu) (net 15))
 (segment (start 209.55 125.222) (end 209.55 129.54) (width 0.254) (layer B.Cu) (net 15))
 (segment (start 208.102204 123.774204) (end 209.55 125.222) (width 0.254) (layer B.Cu) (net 15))
 (segment (start 204.908276 123.774204) (end 208.102204 123.774204) (width 0.254) (layer B.Cu) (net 15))
 (segment (start 203.97794 124.70454) (end 204.908276 123.774204) (width 0.254) (layer B.Cu) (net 15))
 (segment (start 203.97794 125.25686) (end 203.97794 124.70454) (width 0.254) (layer B.Cu) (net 15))
 (segment (start 203.5048 125.73) (end 203.97794 125.25686) (width 0.254) (layer B.Cu) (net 15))
 (segment (start 203.1746 125.73) (end 203.5048 125.73) (width 0.254) (layer B.Cu) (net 15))
 (via (at 203.1746 125.73) (size 0.4572) (layers F.Cu B.Cu) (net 15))
 (segment (start 202.9206 125.73) (end 203.1746 125.73) (width 0.254) (layer F.Cu) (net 15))
 (segment (start 202.67168 125.48108) (end 202.9206 125.73) (width 0.254) (layer F.Cu) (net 15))
 (segment (start 199.63892 123.73102) (end 199.63892 122.16892) (width 0.254) (layer F.Cu) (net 20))
 (segment (start 199.63892 122.16892) (end 199.39 121.92) (width 0.254) (layer F.Cu) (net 20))
 (via (at 200.914 122.936) (size 0.6858) (layers F.Cu B.Cu) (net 18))
 (segment (start 200.63968 123.73102) (end 200.63968 123.21032) (width 0.254) (layer F.Cu) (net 18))
 (segment (start 201.22642 122.936) (end 202.11542 123.825) (width 0.254) (layer F.Cu) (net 18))
 (segment (start 200.914 122.936) (end 201.22642 122.936) (width 0.254) (layer F.Cu) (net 18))
 (segment (start 200.63968 123.21032) (end 200.914 122.936) (width 0.254) (layer F.Cu) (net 18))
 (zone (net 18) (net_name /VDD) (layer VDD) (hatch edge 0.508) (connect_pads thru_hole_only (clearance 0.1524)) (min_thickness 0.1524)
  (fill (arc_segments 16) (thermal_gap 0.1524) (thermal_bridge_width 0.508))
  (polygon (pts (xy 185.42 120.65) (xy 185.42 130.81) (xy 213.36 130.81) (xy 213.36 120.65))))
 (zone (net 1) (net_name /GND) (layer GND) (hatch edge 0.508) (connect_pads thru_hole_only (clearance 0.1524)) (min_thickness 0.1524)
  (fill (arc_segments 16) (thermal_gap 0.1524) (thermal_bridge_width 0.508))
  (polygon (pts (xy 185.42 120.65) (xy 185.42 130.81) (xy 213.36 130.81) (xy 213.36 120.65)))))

